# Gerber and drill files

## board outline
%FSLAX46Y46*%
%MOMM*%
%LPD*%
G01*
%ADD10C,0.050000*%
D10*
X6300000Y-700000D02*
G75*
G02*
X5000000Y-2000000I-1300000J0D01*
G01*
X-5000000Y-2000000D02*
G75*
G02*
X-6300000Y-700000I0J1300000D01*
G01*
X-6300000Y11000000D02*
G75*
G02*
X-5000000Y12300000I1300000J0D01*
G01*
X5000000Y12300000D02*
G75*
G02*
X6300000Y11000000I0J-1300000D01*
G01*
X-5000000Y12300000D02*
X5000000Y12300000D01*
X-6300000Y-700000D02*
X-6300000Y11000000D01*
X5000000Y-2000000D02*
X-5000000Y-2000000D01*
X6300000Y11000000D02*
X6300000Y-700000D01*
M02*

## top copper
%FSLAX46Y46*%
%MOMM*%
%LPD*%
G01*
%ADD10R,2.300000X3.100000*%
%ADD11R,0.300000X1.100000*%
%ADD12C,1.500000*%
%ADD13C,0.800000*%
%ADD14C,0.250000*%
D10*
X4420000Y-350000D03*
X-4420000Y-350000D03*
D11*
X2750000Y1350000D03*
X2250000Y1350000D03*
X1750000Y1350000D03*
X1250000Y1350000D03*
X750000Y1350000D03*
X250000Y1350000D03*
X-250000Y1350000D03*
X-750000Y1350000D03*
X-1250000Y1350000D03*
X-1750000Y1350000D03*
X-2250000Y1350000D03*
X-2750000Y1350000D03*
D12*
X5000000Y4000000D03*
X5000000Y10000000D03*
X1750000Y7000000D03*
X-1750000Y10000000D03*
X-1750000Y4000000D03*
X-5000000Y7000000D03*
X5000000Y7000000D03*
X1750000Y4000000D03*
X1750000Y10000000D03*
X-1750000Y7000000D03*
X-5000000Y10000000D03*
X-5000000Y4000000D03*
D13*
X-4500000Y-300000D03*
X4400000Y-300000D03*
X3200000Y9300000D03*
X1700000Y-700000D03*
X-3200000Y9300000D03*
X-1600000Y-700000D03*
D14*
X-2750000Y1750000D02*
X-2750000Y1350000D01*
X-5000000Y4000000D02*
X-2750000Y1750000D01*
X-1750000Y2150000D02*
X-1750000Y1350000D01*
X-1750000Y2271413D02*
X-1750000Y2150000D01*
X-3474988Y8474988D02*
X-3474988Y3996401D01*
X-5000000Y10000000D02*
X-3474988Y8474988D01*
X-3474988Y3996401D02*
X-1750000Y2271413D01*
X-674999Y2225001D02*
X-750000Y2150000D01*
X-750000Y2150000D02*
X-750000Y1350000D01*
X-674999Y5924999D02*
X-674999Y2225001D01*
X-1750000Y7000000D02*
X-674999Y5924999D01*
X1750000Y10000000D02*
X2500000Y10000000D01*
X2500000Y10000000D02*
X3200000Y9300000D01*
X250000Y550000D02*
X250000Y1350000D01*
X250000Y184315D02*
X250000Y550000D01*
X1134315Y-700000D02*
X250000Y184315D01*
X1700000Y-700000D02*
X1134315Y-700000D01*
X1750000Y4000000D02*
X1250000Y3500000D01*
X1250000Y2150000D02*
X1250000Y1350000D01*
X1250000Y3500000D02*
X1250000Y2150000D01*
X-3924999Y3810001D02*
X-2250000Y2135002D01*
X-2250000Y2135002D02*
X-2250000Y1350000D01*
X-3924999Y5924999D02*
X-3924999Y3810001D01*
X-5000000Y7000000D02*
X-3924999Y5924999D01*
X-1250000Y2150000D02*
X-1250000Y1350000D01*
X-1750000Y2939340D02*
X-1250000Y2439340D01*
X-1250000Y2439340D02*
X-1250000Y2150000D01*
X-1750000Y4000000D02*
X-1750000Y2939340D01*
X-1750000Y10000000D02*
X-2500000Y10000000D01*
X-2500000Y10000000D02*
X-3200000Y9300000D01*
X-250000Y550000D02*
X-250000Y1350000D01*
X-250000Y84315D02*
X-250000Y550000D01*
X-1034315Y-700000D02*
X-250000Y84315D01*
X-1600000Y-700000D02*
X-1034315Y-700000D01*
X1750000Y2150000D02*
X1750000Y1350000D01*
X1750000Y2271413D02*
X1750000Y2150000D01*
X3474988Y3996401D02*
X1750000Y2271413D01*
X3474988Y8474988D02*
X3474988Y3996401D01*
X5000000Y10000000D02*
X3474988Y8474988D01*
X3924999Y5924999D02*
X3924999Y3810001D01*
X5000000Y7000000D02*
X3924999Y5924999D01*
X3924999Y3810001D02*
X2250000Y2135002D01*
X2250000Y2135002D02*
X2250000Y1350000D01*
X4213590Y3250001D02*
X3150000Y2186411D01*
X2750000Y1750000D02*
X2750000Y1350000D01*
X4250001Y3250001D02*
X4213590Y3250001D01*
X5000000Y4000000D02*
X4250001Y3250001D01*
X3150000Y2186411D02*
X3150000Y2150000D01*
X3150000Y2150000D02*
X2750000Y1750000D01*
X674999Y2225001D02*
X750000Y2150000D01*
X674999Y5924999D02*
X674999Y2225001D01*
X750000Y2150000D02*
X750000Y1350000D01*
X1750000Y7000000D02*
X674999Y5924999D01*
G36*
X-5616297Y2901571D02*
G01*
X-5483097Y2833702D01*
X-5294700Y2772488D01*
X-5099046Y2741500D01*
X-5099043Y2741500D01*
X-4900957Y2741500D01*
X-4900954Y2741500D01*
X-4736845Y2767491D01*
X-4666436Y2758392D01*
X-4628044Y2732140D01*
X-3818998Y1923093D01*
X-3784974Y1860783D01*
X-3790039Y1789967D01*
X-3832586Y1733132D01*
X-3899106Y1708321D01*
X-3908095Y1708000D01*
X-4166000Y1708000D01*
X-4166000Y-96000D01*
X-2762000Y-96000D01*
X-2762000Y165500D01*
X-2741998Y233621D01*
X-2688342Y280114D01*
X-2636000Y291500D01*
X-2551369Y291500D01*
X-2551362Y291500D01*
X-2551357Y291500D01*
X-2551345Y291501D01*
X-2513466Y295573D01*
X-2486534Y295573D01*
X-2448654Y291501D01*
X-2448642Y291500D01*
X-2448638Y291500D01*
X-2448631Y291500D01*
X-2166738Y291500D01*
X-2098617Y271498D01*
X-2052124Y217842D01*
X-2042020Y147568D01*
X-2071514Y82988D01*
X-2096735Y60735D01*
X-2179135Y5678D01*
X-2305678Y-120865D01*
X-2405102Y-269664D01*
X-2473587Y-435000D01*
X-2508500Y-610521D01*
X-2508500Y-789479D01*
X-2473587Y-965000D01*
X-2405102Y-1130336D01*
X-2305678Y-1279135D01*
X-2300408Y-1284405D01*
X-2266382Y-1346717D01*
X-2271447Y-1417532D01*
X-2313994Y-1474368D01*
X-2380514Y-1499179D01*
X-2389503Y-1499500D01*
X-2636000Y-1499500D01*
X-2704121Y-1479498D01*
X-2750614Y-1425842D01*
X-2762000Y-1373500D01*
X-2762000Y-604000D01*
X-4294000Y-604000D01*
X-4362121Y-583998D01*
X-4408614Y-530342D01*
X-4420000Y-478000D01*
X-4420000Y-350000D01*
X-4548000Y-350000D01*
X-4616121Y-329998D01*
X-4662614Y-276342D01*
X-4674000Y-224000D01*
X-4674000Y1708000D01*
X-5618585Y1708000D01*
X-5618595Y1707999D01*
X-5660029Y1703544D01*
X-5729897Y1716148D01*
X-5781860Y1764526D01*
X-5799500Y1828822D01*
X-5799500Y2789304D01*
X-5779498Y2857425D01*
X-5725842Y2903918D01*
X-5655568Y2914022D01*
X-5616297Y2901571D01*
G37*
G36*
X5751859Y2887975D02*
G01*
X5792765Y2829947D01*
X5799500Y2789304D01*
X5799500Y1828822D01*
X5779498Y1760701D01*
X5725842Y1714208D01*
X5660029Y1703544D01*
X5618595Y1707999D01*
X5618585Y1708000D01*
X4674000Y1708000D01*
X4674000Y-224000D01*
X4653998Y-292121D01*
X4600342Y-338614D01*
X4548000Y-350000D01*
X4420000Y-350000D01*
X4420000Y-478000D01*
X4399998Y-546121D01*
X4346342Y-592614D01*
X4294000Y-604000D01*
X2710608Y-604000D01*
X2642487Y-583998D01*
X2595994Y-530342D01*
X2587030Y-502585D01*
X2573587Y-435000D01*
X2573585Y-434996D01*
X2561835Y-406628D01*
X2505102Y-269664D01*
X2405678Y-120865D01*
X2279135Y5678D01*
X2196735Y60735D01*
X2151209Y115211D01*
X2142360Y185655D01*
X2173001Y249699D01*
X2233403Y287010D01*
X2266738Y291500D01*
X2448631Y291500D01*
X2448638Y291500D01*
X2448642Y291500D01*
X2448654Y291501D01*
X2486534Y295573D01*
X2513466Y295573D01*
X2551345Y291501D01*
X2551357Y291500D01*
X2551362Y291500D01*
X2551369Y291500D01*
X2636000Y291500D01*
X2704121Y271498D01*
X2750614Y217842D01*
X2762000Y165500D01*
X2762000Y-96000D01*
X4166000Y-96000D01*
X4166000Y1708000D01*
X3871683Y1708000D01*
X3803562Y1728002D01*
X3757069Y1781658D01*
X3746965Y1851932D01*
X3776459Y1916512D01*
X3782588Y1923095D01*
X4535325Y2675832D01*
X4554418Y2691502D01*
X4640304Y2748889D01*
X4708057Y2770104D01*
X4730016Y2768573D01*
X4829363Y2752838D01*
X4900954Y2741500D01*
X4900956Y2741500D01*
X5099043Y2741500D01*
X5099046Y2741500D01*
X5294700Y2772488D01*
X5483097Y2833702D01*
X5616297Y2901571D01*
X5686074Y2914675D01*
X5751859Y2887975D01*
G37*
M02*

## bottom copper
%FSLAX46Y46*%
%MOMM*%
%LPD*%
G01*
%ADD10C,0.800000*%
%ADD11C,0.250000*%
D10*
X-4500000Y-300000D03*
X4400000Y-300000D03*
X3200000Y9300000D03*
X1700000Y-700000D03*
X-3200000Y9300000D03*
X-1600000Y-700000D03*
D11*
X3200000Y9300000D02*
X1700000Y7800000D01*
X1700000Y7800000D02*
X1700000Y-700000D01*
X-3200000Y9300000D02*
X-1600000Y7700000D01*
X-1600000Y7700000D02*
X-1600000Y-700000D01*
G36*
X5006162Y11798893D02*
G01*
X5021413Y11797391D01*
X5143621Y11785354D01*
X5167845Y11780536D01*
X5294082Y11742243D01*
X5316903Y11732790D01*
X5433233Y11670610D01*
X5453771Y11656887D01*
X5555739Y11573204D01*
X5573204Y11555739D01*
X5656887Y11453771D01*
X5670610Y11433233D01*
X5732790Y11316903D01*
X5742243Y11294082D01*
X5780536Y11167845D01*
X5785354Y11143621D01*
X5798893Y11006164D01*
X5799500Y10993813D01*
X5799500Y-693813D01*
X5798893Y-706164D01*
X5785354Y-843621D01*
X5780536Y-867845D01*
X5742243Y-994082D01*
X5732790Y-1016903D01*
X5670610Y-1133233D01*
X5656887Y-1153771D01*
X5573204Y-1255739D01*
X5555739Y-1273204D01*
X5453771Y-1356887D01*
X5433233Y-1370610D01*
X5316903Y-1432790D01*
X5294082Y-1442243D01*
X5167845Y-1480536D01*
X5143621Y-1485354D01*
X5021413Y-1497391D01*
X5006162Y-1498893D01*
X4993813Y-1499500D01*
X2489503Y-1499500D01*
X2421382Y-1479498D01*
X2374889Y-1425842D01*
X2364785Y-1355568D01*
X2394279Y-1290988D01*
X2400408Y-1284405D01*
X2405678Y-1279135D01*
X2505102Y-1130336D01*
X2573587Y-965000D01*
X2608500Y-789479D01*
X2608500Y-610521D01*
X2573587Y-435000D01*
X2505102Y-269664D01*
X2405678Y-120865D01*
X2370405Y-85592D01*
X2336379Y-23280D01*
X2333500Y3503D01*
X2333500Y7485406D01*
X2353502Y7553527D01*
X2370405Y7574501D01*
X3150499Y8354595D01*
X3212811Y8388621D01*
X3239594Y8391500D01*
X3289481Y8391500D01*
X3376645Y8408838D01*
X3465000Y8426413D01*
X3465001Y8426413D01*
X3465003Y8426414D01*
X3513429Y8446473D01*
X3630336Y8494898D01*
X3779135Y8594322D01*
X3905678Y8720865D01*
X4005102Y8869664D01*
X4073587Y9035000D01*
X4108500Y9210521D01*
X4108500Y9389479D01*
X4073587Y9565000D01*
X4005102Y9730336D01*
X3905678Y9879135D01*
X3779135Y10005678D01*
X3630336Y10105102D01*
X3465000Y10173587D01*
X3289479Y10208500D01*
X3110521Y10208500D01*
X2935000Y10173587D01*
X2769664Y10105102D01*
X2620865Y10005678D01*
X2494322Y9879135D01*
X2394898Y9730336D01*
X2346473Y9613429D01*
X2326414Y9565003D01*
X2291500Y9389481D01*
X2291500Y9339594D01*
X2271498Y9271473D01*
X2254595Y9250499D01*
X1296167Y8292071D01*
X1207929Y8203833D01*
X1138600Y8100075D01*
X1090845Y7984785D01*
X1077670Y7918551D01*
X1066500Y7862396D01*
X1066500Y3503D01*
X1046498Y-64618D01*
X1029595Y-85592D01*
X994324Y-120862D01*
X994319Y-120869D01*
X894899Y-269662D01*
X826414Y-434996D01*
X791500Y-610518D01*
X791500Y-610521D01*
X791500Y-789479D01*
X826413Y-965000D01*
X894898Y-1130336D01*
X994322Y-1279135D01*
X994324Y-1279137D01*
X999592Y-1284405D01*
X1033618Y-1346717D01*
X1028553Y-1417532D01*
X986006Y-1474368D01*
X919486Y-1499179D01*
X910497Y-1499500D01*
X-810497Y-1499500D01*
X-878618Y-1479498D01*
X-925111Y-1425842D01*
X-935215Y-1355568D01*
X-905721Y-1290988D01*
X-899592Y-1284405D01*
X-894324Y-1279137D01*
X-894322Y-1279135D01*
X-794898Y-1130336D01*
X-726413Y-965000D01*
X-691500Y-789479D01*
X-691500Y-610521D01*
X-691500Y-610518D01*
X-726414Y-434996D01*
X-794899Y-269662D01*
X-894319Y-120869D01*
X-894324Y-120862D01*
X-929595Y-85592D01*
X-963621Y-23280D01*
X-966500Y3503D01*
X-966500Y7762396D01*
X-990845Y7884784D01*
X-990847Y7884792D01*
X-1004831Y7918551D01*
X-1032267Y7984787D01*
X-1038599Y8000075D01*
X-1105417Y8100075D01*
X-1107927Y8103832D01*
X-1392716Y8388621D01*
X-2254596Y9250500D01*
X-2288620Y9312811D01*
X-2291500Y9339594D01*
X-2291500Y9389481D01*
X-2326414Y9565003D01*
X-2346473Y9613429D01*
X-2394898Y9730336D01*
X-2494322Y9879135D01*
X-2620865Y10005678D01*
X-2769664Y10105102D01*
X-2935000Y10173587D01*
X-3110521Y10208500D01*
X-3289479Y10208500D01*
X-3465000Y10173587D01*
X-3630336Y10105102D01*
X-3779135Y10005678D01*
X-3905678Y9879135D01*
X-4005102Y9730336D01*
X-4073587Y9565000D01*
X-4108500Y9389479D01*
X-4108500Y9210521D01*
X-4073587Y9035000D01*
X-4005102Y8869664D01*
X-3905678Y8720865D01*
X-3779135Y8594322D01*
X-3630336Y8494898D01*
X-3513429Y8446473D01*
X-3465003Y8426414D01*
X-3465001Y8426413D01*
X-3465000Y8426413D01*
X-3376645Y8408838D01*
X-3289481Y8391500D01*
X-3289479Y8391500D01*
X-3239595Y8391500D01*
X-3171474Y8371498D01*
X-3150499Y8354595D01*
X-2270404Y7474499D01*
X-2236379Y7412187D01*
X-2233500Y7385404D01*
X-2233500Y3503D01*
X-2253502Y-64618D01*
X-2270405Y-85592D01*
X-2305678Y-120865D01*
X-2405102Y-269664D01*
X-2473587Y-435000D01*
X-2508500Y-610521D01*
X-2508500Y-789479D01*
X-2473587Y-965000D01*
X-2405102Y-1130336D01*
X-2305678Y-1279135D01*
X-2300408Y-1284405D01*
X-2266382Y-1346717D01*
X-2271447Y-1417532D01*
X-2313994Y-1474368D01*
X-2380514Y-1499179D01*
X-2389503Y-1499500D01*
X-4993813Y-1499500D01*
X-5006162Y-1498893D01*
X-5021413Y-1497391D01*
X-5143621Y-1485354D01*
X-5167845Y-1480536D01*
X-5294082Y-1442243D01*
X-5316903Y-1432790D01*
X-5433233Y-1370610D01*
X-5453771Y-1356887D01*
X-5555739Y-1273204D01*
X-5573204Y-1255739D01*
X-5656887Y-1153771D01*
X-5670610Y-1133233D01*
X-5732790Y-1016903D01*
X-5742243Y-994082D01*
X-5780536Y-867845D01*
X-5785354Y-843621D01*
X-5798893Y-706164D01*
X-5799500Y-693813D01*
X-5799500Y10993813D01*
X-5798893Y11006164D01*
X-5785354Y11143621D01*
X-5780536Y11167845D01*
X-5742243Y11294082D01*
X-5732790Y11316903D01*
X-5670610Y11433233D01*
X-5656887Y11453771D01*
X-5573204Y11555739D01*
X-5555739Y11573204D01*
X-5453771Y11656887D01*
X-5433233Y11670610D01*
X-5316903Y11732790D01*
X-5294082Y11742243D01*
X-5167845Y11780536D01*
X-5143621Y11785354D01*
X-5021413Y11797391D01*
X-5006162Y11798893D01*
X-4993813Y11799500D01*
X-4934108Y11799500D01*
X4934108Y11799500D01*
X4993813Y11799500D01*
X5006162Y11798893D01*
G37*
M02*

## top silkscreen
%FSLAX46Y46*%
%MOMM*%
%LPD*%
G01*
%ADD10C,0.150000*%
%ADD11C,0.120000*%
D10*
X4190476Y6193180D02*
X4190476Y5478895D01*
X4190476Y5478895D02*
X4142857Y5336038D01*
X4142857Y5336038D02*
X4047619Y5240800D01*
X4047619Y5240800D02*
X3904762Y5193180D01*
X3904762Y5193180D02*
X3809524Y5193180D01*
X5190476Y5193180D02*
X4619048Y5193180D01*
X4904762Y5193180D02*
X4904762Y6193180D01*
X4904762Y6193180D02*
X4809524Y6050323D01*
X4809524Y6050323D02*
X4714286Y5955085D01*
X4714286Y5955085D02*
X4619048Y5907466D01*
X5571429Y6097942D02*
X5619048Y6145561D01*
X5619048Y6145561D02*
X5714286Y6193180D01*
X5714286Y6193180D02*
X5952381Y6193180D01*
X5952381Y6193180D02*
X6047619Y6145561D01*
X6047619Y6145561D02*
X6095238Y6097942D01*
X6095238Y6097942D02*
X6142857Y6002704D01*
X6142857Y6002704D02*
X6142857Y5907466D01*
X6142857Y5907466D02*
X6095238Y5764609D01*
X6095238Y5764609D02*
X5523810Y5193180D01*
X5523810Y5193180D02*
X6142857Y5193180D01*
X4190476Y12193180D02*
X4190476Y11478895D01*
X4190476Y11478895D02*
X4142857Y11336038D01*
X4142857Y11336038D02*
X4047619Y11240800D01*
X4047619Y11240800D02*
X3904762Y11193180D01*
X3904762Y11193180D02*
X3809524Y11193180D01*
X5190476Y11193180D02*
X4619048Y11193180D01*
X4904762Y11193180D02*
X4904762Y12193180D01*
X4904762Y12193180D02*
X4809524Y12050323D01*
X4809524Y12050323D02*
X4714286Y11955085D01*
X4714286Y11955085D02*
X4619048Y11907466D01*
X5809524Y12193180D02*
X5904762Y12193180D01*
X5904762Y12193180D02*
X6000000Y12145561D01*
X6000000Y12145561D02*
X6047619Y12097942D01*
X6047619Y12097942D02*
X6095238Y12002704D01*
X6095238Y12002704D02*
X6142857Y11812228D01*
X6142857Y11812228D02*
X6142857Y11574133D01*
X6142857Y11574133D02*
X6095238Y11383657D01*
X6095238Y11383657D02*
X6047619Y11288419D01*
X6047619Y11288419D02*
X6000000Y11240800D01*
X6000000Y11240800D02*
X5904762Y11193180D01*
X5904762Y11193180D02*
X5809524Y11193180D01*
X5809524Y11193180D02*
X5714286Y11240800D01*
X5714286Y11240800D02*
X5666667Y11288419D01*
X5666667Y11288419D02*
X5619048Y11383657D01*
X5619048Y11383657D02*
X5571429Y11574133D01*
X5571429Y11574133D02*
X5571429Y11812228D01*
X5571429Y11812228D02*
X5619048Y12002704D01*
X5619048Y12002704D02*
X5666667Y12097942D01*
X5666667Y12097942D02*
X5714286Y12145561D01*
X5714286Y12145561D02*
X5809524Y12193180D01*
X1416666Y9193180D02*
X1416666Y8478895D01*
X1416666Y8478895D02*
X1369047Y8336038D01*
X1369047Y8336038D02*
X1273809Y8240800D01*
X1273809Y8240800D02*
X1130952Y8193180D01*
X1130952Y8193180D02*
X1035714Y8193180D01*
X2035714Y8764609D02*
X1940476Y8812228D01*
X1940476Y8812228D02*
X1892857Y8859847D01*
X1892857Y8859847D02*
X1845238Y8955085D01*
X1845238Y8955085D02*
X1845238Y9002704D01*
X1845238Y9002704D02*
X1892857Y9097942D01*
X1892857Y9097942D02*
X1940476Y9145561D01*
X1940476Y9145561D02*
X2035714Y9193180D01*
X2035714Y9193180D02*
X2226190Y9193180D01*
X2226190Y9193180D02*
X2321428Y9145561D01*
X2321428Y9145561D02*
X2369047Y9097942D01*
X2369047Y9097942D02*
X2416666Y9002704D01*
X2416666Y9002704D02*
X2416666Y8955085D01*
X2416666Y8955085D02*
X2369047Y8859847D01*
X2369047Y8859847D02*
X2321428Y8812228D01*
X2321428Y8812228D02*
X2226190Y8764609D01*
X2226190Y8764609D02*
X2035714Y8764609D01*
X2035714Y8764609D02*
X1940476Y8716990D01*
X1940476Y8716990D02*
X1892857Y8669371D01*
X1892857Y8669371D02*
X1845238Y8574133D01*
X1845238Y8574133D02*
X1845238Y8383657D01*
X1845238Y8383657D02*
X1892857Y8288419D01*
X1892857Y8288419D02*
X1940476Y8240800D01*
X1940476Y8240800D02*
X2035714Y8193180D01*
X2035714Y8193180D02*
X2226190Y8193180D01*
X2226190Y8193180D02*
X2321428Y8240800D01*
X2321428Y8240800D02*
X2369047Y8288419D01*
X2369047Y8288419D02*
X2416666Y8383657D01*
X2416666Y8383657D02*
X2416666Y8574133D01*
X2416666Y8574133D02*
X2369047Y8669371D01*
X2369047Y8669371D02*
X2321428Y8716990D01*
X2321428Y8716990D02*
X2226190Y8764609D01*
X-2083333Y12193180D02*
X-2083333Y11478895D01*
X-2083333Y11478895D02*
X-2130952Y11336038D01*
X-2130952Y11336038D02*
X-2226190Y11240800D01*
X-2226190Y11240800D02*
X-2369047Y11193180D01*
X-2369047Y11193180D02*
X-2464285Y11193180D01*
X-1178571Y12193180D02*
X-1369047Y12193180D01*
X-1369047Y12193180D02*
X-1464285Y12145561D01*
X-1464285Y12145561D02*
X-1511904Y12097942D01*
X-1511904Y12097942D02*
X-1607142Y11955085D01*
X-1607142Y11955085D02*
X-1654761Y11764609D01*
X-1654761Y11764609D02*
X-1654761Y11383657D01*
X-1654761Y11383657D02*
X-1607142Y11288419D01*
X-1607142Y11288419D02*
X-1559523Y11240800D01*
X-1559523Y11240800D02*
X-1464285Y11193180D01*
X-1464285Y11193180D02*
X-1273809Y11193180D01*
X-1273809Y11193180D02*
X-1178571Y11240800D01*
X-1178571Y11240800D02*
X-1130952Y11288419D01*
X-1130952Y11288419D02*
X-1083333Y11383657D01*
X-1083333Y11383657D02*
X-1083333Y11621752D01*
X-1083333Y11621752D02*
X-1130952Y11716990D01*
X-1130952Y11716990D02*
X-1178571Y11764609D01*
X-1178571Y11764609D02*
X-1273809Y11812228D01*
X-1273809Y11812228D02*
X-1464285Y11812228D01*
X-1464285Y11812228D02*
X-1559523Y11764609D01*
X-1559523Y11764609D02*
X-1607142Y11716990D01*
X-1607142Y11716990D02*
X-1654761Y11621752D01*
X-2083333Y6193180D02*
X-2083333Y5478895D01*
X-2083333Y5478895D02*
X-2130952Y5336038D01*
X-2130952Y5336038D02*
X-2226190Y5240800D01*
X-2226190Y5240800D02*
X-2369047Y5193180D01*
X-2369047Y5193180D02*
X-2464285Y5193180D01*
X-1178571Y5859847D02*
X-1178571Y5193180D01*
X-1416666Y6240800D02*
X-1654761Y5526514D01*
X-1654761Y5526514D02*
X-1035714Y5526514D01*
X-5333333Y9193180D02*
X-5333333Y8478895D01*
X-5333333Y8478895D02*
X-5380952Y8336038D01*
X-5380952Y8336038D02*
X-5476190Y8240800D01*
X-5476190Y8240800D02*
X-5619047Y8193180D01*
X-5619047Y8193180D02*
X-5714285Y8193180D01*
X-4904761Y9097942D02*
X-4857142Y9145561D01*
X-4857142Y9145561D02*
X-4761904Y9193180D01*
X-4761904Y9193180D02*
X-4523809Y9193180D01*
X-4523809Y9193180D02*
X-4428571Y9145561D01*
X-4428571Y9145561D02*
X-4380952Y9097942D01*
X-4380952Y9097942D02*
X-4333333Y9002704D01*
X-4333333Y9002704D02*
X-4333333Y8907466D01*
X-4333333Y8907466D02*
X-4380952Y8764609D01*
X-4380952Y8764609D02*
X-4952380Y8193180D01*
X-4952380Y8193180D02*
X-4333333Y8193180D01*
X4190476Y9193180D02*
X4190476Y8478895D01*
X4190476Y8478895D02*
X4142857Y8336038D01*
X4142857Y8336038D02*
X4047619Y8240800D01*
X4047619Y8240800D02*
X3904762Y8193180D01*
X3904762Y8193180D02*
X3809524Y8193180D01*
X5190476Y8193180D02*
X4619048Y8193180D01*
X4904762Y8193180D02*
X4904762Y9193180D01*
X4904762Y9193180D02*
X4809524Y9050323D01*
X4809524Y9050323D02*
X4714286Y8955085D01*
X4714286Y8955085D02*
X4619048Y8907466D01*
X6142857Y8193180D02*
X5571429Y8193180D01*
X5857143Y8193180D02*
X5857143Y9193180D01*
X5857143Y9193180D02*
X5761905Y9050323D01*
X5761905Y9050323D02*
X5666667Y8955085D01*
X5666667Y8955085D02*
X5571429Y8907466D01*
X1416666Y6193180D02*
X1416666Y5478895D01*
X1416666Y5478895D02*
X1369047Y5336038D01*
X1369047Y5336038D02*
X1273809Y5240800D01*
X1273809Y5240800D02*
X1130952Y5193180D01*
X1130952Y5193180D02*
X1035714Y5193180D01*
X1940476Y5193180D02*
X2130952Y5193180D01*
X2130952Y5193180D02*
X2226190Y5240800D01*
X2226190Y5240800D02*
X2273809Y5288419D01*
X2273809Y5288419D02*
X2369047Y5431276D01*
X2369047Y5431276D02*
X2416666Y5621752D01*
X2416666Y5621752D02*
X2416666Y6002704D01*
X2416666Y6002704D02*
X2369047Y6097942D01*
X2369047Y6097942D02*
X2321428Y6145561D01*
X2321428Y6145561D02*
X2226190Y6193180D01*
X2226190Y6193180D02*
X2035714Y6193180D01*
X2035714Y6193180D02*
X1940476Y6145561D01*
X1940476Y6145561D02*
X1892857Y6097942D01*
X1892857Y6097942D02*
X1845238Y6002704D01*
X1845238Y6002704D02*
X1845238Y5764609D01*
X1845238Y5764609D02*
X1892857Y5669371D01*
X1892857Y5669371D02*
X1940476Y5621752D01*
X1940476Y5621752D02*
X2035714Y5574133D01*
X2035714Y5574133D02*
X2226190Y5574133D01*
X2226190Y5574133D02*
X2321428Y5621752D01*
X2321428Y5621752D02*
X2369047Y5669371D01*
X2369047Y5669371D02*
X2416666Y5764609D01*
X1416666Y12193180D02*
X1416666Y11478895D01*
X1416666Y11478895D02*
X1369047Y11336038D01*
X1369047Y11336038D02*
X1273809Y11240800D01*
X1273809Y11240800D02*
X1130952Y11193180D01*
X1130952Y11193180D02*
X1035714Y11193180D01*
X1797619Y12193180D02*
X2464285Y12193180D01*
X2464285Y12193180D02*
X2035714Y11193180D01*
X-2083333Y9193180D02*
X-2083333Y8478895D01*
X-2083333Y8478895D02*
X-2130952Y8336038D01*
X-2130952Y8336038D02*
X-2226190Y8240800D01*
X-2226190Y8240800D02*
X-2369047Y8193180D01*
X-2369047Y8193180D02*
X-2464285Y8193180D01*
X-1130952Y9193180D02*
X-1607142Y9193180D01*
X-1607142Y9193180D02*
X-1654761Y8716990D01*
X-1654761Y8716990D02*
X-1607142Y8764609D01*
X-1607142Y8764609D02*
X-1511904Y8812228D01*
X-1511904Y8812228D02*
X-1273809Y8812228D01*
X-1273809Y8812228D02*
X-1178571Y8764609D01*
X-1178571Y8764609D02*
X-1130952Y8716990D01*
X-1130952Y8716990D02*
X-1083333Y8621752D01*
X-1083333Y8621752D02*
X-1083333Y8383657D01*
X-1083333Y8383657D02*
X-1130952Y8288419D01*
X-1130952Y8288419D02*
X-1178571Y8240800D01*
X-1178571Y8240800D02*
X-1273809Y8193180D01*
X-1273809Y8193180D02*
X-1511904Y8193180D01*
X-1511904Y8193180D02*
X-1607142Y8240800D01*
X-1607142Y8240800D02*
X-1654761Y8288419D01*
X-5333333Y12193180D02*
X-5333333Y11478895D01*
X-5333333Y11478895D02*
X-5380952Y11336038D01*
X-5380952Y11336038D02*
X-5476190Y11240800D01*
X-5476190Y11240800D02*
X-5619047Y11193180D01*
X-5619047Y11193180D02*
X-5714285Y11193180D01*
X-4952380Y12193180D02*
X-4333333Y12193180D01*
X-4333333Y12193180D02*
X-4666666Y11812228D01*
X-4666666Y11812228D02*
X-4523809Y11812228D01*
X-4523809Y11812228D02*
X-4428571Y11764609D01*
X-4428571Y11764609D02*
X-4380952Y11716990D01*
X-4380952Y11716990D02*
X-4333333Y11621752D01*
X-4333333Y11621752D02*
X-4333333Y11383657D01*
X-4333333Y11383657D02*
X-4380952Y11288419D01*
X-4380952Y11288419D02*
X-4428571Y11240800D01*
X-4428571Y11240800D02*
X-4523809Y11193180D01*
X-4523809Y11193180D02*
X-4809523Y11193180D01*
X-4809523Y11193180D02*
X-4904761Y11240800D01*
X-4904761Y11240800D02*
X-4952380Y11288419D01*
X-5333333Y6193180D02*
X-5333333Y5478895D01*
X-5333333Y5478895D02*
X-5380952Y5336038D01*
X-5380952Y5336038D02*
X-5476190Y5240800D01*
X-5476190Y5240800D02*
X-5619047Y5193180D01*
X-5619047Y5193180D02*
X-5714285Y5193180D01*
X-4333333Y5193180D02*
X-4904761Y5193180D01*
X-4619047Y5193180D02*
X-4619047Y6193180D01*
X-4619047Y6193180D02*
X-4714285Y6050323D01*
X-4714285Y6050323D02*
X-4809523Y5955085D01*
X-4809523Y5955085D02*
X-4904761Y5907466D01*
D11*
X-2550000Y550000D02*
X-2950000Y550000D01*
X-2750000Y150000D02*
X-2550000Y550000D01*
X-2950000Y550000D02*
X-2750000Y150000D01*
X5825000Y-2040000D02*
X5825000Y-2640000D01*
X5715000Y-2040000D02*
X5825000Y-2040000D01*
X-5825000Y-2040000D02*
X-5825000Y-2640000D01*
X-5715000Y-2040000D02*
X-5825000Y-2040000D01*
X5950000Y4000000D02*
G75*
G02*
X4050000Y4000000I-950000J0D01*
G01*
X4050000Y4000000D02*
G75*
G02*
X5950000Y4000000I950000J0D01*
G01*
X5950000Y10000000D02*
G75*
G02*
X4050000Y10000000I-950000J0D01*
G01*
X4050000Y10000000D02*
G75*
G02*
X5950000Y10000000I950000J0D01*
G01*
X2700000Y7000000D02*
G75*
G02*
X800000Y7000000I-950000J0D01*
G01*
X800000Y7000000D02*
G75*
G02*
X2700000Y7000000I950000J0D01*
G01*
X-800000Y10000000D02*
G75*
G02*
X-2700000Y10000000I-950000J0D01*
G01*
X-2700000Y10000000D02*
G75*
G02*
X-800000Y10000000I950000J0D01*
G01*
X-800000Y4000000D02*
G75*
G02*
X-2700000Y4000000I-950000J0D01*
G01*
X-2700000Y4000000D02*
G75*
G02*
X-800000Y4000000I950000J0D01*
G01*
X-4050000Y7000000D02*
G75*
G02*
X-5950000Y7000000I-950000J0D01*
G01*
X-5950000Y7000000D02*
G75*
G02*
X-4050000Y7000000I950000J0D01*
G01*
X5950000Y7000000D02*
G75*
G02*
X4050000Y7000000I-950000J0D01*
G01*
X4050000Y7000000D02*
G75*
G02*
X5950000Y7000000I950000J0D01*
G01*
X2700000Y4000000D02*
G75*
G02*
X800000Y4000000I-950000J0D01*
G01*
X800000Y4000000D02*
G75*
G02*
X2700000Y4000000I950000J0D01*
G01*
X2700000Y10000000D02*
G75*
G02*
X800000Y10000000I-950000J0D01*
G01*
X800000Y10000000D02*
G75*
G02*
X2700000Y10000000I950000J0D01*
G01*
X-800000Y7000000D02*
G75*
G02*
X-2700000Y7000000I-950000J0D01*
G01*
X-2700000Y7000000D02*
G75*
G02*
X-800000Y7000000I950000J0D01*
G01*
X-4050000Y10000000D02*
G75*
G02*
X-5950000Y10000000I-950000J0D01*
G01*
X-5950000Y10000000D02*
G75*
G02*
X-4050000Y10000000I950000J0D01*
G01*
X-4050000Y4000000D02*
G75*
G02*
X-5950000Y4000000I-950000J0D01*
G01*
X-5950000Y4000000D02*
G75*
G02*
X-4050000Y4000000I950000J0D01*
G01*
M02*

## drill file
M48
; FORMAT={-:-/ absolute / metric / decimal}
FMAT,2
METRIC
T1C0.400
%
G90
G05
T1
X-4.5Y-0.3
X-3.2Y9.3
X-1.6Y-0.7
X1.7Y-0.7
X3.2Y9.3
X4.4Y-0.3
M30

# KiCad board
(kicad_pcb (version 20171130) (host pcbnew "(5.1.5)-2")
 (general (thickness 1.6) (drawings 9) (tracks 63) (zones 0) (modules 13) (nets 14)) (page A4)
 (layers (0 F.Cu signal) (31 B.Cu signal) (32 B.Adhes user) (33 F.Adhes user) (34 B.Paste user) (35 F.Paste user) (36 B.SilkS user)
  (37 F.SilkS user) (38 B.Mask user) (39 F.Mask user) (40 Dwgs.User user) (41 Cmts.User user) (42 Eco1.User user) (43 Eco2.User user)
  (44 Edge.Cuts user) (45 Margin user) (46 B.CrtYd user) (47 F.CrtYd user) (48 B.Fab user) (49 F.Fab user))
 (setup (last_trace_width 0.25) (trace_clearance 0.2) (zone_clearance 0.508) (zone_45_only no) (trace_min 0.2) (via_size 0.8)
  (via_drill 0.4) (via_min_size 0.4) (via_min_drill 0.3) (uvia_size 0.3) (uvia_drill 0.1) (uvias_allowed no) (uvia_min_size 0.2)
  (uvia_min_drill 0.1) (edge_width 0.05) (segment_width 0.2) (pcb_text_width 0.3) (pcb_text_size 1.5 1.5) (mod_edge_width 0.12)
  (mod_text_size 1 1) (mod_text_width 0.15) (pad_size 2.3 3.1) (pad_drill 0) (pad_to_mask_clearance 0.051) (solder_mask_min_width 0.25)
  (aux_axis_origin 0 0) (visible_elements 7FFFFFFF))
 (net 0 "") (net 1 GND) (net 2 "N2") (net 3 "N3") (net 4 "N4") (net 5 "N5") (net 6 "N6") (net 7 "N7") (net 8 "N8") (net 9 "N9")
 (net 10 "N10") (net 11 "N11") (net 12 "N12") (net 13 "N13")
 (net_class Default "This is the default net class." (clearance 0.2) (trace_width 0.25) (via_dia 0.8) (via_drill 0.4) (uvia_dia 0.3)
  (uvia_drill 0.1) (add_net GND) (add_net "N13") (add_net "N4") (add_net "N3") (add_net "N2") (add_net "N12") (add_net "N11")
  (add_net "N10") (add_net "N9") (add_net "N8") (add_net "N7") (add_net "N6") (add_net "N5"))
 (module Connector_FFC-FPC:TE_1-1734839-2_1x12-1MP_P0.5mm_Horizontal (layer F.Cu) (at 0 0)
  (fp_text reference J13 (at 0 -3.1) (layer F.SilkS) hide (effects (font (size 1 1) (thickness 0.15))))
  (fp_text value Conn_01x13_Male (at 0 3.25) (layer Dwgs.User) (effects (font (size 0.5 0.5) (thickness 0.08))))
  (fp_line (start -2.55 -0.55) (end -2.95 -0.55) (layer F.SilkS) (width 0.12))
  (fp_line (start -2.75 -0.15) (end -2.55 -0.55) (layer F.SilkS) (width 0.12))
  (fp_line (start -2.95 -0.55) (end -2.75 -0.15) (layer F.SilkS) (width 0.12))
  (fp_line (start 5.825 2.04) (end 5.825 2.64) (layer F.SilkS) (width 0.12))
  (fp_line (start 5.715 2.04) (end 5.825 2.04) (layer F.SilkS) (width 0.12))
  (fp_line (start -5.825 2.04) (end -5.825 2.64) (layer F.SilkS) (width 0.12))
  (fp_line (start -5.715 2.04) (end -5.825 2.04) (layer F.SilkS) (width 0.12))
  (pad 13 smd rect (at 4.42 0.35) (size 2.3 3.1) (layers F.Cu F.Paste F.Mask) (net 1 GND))
  (pad 13 smd rect (at -4.42 0.35) (size 2.3 3.1) (layers F.Cu F.Paste F.Mask) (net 1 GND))
  (pad 12 smd rect (at 2.75 -1.35) (size 0.3 1.1) (layers F.Cu F.Paste F.Mask) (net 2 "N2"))
  (pad 11 smd rect (at 2.25 -1.35) (size 0.3 1.1) (layers F.Cu F.Paste F.Mask) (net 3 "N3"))
  (pad 10 smd rect (at 1.75 -1.35) (size 0.3 1.1) (layers F.Cu F.Paste F.Mask) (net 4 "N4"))
  (pad 9 smd rect (at 1.25 -1.35) (size 0.3 1.1) (layers F.Cu F.Paste F.Mask) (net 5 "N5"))
  (pad 8 smd rect (at 0.75 -1.35) (size 0.3 1.1) (layers F.Cu F.Paste F.Mask) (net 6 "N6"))
  (pad 7 smd rect (at 0.25 -1.35) (size 0.3 1.1) (layers F.Cu F.Paste F.Mask) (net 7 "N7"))
  (pad 6 smd rect (at -0.25 -1.35) (size 0.3 1.1) (layers F.Cu F.Paste F.Mask) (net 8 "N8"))
  (pad 5 smd rect (at -0.75 -1.35) (size 0.3 1.1) (layers F.Cu F.Paste F.Mask) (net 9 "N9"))
  (pad 4 smd rect (at -1.25 -1.35) (size 0.3 1.1) (layers F.Cu F.Paste F.Mask) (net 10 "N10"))
  (pad 3 smd rect (at -1.75 -1.35) (size 0.3 1.1) (layers F.Cu F.Paste F.Mask) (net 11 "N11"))
  (pad 2 smd rect (at -2.25 -1.35) (size 0.3 1.1) (layers F.Cu F.Paste F.Mask) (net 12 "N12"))
  (pad 1 smd rect (at -2.75 -1.35) (size 0.3 1.1) (layers F.Cu F.Paste F.Mask) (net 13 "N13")))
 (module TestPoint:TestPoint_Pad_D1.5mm (layer F.Cu) (at 5 -4)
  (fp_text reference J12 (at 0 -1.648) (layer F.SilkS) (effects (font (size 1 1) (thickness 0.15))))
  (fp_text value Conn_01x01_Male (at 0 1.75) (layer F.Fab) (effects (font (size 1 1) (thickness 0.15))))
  (fp_circle (center 0 0) (end 0 0.95) (layer F.SilkS) (width 0.12))
  (pad 1 smd circle (at 0 0) (size 1.5 1.5) (layers F.Cu F.Mask) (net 2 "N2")))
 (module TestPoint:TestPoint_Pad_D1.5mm (layer F.Cu) (at 5 -10)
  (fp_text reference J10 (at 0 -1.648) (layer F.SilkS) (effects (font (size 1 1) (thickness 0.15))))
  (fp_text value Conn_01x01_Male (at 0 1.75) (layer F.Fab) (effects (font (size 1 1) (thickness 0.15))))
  (fp_circle (center 0 0) (end 0 0.95) (layer F.SilkS) (width 0.12))
  (pad 1 smd circle (at 0 0) (size 1.5 1.5) (layers F.Cu F.Mask) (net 4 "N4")))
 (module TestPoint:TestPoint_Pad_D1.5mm (layer F.Cu) (at 1.75 -7)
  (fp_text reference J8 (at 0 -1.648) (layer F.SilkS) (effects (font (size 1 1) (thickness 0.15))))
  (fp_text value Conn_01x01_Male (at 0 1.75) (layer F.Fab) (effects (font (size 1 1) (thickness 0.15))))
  (fp_circle (center 0 0) (end 0 0.95) (layer F.SilkS) (width 0.12))
  (pad 1 smd circle (at 0 0) (size 1.5 1.5) (layers F.Cu F.Mask) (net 6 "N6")))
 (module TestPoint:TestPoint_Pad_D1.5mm (layer F.Cu) (at -1.75 -10)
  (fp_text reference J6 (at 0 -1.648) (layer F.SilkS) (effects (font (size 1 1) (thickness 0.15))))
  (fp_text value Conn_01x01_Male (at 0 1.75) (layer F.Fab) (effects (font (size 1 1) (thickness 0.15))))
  (fp_circle (center 0 0) (end 0 0.95) (layer F.SilkS) (width 0.12))
  (pad 1 smd circle (at 0 0) (size 1.5 1.5) (layers F.Cu F.Mask) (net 8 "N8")))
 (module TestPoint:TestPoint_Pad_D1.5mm (layer F.Cu) (at -1.75 -4)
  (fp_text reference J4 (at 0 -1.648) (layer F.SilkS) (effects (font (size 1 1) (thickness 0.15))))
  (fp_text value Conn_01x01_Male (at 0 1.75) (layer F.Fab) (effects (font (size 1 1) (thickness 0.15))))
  (fp_circle (center 0 0) (end 0 0.95) (layer F.SilkS) (width 0.12))
  (pad 1 smd circle (at 0 0) (size 1.5 1.5) (layers F.Cu F.Mask) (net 10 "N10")))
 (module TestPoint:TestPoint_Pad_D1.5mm (layer F.Cu) (at -5 -7)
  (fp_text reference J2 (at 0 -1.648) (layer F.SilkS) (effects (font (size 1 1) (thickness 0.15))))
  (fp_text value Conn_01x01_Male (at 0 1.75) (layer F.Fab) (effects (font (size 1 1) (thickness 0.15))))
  (fp_circle (center 0 0) (end 0 0.95) (layer F.SilkS) (width 0.12))
  (pad 1 smd circle (at 0 0) (size 1.5 1.5) (layers F.Cu F.Mask) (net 12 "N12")))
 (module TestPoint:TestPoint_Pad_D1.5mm (layer F.Cu) (at 5 -7)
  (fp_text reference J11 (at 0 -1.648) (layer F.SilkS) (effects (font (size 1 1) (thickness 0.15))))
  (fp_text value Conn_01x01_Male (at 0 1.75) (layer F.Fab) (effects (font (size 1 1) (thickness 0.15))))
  (fp_circle (center 0 0) (end 0 0.95) (layer F.SilkS) (width 0.12))
  (pad 1 smd circle (at 0 0) (size 1.5 1.5) (layers F.Cu F.Mask) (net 3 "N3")))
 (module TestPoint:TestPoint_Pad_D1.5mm (layer F.Cu) (at 1.75 -4)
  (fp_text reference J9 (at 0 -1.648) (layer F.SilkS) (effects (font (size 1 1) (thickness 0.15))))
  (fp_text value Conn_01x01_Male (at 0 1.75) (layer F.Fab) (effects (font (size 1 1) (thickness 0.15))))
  (fp_circle (center 0 0) (end 0 0.95) (layer F.SilkS) (width 0.12))
  (pad 1 smd circle (at 0 0) (size 1.5 1.5) (layers F.Cu F.Mask) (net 5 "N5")))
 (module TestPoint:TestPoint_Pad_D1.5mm (layer F.Cu) (at 1.75 -10)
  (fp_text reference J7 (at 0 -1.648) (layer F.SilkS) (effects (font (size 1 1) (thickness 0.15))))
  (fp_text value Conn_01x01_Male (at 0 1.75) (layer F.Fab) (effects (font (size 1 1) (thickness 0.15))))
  (fp_circle (center 0 0) (end 0 0.95) (layer F.SilkS) (width 0.12))
  (pad 1 smd circle (at 0 0) (size 1.5 1.5) (layers F.Cu F.Mask) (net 7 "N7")))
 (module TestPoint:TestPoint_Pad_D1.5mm (layer F.Cu) (at -1.75 -7)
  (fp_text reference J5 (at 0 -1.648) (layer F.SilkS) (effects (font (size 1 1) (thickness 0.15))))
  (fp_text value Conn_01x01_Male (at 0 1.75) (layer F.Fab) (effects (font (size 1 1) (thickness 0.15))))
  (fp_circle (center 0 0) (end 0 0.95) (layer F.SilkS) (width 0.12))
  (pad 1 smd circle (at 0 0) (size 1.5 1.5) (layers F.Cu F.Mask) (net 9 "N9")))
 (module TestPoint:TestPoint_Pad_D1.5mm (layer F.Cu) (at -5 -10)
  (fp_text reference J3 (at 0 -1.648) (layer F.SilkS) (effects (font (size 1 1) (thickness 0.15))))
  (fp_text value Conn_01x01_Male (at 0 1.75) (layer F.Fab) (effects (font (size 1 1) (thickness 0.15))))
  (fp_circle (center 0 0) (end 0 0.95) (layer F.SilkS) (width 0.12))
  (pad 1 smd circle (at 0 0) (size 1.5 1.5) (layers F.Cu F.Mask) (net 11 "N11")))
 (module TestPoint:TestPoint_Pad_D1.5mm (layer F.Cu) (at -5 -4)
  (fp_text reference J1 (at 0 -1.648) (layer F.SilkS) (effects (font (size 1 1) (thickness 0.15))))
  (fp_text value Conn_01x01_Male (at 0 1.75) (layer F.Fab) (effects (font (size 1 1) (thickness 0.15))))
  (fp_circle (center 0 0) (end 0 0.95) (layer F.SilkS) (width 0.12))
  (pad 1 smd circle (at 0 0) (size 1.5 1.5) (layers F.Cu F.Mask) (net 13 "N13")))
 (gr_arc (start 5 0.7) (end 5 2) (angle -90) (layer Edge.Cuts) (width 0.05))
 (gr_arc (start -5 0.7) (end -6.3 0.7) (angle -90) (layer Edge.Cuts) (width 0.05))
 (gr_arc (start -5 -11) (end -5 -12.3) (angle -90) (layer Edge.Cuts) (width 0.05))
 (gr_arc (start 5 -11) (end 6.3 -11) (angle -90) (layer Edge.Cuts) (width 0.05))
 (gr_line (start -5 -12.3) (end 5 -12.3) (layer Edge.Cuts) (width 0.05))
 (gr_line (start -6.3 0.7) (end -6.3 -11) (layer Edge.Cuts) (width 0.05))
 (gr_line (start 5 2) (end -5 2) (layer Edge.Cuts) (width 0.05))
 (gr_line (start 6.3 -11) (end 6.3 0.7) (layer Edge.Cuts) (width 0.05))
 (via (at -4.5 0.3) (size 0.8) (drill 0.4) (layers F.Cu B.Cu) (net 1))
 (via (at 4.4 0.3) (size 0.8) (drill 0.4) (layers F.Cu B.Cu) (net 1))
 (segment (start -2.75 -1.75) (end -2.75 -1.35) (width 0.25) (layer F.Cu) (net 13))
 (segment (start -5 -4) (end -2.75 -1.75) (width 0.25) (layer F.Cu) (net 13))
 (segment (start -1.75 -2.15) (end -1.75 -1.35) (width 0.25) (layer F.Cu) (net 11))
 (segment (start -1.75 -2.271413) (end -1.75 -2.15) (width 0.25) (layer F.Cu) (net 11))
 (segment (start -3.474988 -8.474988) (end -3.474988 -3.996401) (width 0.25) (layer F.Cu) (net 11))
 (segment (start -5 -10) (end -3.474988 -8.474988) (width 0.25) (layer F.Cu) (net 11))
 (segment (start -3.474988 -3.996401) (end -1.75 -2.271413) (width 0.25) (layer F.Cu) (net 11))
 (segment (start -0.674999 -2.225001) (end -0.75 -2.15) (width 0.25) (layer F.Cu) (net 9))
 (segment (start -0.75 -2.15) (end -0.75 -1.35) (width 0.25) (layer F.Cu) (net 9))
 (segment (start -0.674999 -5.924999) (end -0.674999 -2.225001) (width 0.25) (layer F.Cu) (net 9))
 (segment (start -1.75 -7) (end -0.674999 -5.924999) (width 0.25) (layer F.Cu) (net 9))
 (via (at 3.2 -9.3) (size 0.8) (drill 0.4) (layers F.Cu B.Cu) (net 7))
 (segment (start 1.75 -10) (end 2.5 -10) (width 0.25) (layer F.Cu) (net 7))
 (segment (start 2.5 -10) (end 3.2 -9.3) (width 0.25) (layer F.Cu) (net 7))
 (segment (start 3.2 -9.3) (end 1.7 -7.8) (width 0.25) (layer B.Cu) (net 7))
 (via (at 1.7 0.7) (size 0.8) (drill 0.4) (layers F.Cu B.Cu) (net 7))
 (segment (start 1.7 -7.8) (end 1.7 0.7) (width 0.25) (layer B.Cu) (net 7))
 (segment (start 0.25 -0.55) (end 0.25 -1.35) (width 0.25) (layer F.Cu) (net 7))
 (segment (start 0.25 -0.184315) (end 0.25 -0.55) (width 0.25) (layer F.Cu) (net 7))
 (segment (start 1.134315 0.7) (end 0.25 -0.184315) (width 0.25) (layer F.Cu) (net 7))
 (segment (start 1.7 0.7) (end 1.134315 0.7) (width 0.25) (layer F.Cu) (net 7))
 (segment (start 1.75 -4) (end 1.25 -3.5) (width 0.25) (layer F.Cu) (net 5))
 (segment (start 1.25 -2.15) (end 1.25 -1.35) (width 0.25) (layer F.Cu) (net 5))
 (segment (start 1.25 -3.5) (end 1.25 -2.15) (width 0.25) (layer F.Cu) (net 5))
 (segment (start -3.924999 -3.810001) (end -2.25 -2.135002) (width 0.25) (layer F.Cu) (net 12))
 (segment (start -2.25 -2.135002) (end -2.25 -1.35) (width 0.25) (layer F.Cu) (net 12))
 (segment (start -3.924999 -5.924999) (end -3.924999 -3.810001) (width 0.25) (layer F.Cu) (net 12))
 (segment (start -5 -7) (end -3.924999 -5.924999) (width 0.25) (layer F.Cu) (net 12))
 (segment (start -1.25 -2.15) (end -1.25 -1.35) (width 0.25) (layer F.Cu) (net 10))
 (segment (start -1.75 -2.93934) (end -1.25 -2.43934) (width 0.25) (layer F.Cu) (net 10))
 (segment (start -1.25 -2.43934) (end -1.25 -2.15) (width 0.25) (layer F.Cu) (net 10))
 (segment (start -1.75 -4) (end -1.75 -2.93934) (width 0.25) (layer F.Cu) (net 10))
 (via (at -3.2 -9.3) (size 0.8) (drill 0.4) (layers F.Cu B.Cu) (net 8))
 (segment (start -1.75 -10) (end -2.5 -10) (width 0.25) (layer F.Cu) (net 8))
 (segment (start -2.5 -10) (end -3.2 -9.3) (width 0.25) (layer F.Cu) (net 8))
 (via (at -1.6 0.7) (size 0.8) (drill 0.4) (layers F.Cu B.Cu) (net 8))
 (segment (start -3.2 -9.3) (end -1.6 -7.7) (width 0.25) (layer B.Cu) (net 8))
 (segment (start -1.6 -7.7) (end -1.6 0.7) (width 0.25) (layer B.Cu) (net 8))
 (segment (start -0.25 -0.55) (end -0.25 -1.35) (width 0.25) (layer F.Cu) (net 8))
 (segment (start -0.25 -0.084315) (end -0.25 -0.55) (width 0.25) (layer F.Cu) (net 8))
 (segment (start -1.034315 0.7) (end -0.25 -0.084315) (width 0.25) (layer F.Cu) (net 8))
 (segment (start -1.6 0.7) (end -1.034315 0.7) (width 0.25) (layer F.Cu) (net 8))
 (segment (start 1.75 -2.15) (end 1.75 -1.35) (width 0.25) (layer F.Cu) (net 4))
 (segment (start 1.75 -2.271413) (end 1.75 -2.15) (width 0.25) (layer F.Cu) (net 4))
 (segment (start 3.474988 -3.996401) (end 1.75 -2.271413) (width 0.25) (layer F.Cu) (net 4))
 (segment (start 3.474988 -8.474988) (end 3.474988 -3.996401) (width 0.25) (layer F.Cu) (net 4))
 (segment (start 5 -10) (end 3.474988 -8.474988) (width 0.25) (layer F.Cu) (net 4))
 (segment (start 3.924999 -5.924999) (end 3.924999 -3.810001) (width 0.25) (layer F.Cu) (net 3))
 (segment (start 5 -7) (end 3.924999 -5.924999) (width 0.25) (layer F.Cu) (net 3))
 (segment (start 3.924999 -3.810001) (end 2.25 -2.135002) (width 0.25) (layer F.Cu) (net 3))
 (segment (start 2.25 -2.135002) (end 2.25 -1.35) (width 0.25) (layer F.Cu) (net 3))
 (segment (start 4.21359 -3.250001) (end 3.15 -2.186411) (width 0.25) (layer F.Cu) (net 2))
 (segment (start 2.75 -1.75) (end 2.75 -1.35) (width 0.25) (layer F.Cu) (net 2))
 (segment (start 4.250001 -3.250001) (end 4.21359 -3.250001) (width 0.25) (layer F.Cu) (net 2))
 (segment (start 5 -4) (end 4.250001 -3.250001) (width 0.25) (layer F.Cu) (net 2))
 (segment (start 3.15 -2.186411) (end 3.15 -2.15) (width 0.25) (layer F.Cu) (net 2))
 (segment (start 3.15 -2.15) (end 2.75 -1.75) (width 0.25) (layer F.Cu) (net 2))
 (segment (start 0.674999 -2.225001) (end 0.75 -2.15) (width 0.25) (layer F.Cu) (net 6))
 (segment (start 0.674999 -5.924999) (end 0.674999 -2.225001) (width 0.25) (layer F.Cu) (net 6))
 (segment (start 0.75 -2.15) (end 0.75 -1.35) (width 0.25) (layer F.Cu) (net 6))
 (segment (start 1.75 -7) (end 0.674999 -5.924999) (width 0.25) (layer F.Cu) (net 6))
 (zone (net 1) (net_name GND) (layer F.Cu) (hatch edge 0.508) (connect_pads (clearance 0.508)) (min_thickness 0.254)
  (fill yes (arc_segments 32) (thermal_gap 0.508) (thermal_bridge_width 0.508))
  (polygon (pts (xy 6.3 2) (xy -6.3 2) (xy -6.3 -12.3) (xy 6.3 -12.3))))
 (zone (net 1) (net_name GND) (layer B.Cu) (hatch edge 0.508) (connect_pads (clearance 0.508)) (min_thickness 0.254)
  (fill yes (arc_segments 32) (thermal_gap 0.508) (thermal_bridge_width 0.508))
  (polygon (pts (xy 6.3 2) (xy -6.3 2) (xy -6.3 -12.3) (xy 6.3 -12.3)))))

